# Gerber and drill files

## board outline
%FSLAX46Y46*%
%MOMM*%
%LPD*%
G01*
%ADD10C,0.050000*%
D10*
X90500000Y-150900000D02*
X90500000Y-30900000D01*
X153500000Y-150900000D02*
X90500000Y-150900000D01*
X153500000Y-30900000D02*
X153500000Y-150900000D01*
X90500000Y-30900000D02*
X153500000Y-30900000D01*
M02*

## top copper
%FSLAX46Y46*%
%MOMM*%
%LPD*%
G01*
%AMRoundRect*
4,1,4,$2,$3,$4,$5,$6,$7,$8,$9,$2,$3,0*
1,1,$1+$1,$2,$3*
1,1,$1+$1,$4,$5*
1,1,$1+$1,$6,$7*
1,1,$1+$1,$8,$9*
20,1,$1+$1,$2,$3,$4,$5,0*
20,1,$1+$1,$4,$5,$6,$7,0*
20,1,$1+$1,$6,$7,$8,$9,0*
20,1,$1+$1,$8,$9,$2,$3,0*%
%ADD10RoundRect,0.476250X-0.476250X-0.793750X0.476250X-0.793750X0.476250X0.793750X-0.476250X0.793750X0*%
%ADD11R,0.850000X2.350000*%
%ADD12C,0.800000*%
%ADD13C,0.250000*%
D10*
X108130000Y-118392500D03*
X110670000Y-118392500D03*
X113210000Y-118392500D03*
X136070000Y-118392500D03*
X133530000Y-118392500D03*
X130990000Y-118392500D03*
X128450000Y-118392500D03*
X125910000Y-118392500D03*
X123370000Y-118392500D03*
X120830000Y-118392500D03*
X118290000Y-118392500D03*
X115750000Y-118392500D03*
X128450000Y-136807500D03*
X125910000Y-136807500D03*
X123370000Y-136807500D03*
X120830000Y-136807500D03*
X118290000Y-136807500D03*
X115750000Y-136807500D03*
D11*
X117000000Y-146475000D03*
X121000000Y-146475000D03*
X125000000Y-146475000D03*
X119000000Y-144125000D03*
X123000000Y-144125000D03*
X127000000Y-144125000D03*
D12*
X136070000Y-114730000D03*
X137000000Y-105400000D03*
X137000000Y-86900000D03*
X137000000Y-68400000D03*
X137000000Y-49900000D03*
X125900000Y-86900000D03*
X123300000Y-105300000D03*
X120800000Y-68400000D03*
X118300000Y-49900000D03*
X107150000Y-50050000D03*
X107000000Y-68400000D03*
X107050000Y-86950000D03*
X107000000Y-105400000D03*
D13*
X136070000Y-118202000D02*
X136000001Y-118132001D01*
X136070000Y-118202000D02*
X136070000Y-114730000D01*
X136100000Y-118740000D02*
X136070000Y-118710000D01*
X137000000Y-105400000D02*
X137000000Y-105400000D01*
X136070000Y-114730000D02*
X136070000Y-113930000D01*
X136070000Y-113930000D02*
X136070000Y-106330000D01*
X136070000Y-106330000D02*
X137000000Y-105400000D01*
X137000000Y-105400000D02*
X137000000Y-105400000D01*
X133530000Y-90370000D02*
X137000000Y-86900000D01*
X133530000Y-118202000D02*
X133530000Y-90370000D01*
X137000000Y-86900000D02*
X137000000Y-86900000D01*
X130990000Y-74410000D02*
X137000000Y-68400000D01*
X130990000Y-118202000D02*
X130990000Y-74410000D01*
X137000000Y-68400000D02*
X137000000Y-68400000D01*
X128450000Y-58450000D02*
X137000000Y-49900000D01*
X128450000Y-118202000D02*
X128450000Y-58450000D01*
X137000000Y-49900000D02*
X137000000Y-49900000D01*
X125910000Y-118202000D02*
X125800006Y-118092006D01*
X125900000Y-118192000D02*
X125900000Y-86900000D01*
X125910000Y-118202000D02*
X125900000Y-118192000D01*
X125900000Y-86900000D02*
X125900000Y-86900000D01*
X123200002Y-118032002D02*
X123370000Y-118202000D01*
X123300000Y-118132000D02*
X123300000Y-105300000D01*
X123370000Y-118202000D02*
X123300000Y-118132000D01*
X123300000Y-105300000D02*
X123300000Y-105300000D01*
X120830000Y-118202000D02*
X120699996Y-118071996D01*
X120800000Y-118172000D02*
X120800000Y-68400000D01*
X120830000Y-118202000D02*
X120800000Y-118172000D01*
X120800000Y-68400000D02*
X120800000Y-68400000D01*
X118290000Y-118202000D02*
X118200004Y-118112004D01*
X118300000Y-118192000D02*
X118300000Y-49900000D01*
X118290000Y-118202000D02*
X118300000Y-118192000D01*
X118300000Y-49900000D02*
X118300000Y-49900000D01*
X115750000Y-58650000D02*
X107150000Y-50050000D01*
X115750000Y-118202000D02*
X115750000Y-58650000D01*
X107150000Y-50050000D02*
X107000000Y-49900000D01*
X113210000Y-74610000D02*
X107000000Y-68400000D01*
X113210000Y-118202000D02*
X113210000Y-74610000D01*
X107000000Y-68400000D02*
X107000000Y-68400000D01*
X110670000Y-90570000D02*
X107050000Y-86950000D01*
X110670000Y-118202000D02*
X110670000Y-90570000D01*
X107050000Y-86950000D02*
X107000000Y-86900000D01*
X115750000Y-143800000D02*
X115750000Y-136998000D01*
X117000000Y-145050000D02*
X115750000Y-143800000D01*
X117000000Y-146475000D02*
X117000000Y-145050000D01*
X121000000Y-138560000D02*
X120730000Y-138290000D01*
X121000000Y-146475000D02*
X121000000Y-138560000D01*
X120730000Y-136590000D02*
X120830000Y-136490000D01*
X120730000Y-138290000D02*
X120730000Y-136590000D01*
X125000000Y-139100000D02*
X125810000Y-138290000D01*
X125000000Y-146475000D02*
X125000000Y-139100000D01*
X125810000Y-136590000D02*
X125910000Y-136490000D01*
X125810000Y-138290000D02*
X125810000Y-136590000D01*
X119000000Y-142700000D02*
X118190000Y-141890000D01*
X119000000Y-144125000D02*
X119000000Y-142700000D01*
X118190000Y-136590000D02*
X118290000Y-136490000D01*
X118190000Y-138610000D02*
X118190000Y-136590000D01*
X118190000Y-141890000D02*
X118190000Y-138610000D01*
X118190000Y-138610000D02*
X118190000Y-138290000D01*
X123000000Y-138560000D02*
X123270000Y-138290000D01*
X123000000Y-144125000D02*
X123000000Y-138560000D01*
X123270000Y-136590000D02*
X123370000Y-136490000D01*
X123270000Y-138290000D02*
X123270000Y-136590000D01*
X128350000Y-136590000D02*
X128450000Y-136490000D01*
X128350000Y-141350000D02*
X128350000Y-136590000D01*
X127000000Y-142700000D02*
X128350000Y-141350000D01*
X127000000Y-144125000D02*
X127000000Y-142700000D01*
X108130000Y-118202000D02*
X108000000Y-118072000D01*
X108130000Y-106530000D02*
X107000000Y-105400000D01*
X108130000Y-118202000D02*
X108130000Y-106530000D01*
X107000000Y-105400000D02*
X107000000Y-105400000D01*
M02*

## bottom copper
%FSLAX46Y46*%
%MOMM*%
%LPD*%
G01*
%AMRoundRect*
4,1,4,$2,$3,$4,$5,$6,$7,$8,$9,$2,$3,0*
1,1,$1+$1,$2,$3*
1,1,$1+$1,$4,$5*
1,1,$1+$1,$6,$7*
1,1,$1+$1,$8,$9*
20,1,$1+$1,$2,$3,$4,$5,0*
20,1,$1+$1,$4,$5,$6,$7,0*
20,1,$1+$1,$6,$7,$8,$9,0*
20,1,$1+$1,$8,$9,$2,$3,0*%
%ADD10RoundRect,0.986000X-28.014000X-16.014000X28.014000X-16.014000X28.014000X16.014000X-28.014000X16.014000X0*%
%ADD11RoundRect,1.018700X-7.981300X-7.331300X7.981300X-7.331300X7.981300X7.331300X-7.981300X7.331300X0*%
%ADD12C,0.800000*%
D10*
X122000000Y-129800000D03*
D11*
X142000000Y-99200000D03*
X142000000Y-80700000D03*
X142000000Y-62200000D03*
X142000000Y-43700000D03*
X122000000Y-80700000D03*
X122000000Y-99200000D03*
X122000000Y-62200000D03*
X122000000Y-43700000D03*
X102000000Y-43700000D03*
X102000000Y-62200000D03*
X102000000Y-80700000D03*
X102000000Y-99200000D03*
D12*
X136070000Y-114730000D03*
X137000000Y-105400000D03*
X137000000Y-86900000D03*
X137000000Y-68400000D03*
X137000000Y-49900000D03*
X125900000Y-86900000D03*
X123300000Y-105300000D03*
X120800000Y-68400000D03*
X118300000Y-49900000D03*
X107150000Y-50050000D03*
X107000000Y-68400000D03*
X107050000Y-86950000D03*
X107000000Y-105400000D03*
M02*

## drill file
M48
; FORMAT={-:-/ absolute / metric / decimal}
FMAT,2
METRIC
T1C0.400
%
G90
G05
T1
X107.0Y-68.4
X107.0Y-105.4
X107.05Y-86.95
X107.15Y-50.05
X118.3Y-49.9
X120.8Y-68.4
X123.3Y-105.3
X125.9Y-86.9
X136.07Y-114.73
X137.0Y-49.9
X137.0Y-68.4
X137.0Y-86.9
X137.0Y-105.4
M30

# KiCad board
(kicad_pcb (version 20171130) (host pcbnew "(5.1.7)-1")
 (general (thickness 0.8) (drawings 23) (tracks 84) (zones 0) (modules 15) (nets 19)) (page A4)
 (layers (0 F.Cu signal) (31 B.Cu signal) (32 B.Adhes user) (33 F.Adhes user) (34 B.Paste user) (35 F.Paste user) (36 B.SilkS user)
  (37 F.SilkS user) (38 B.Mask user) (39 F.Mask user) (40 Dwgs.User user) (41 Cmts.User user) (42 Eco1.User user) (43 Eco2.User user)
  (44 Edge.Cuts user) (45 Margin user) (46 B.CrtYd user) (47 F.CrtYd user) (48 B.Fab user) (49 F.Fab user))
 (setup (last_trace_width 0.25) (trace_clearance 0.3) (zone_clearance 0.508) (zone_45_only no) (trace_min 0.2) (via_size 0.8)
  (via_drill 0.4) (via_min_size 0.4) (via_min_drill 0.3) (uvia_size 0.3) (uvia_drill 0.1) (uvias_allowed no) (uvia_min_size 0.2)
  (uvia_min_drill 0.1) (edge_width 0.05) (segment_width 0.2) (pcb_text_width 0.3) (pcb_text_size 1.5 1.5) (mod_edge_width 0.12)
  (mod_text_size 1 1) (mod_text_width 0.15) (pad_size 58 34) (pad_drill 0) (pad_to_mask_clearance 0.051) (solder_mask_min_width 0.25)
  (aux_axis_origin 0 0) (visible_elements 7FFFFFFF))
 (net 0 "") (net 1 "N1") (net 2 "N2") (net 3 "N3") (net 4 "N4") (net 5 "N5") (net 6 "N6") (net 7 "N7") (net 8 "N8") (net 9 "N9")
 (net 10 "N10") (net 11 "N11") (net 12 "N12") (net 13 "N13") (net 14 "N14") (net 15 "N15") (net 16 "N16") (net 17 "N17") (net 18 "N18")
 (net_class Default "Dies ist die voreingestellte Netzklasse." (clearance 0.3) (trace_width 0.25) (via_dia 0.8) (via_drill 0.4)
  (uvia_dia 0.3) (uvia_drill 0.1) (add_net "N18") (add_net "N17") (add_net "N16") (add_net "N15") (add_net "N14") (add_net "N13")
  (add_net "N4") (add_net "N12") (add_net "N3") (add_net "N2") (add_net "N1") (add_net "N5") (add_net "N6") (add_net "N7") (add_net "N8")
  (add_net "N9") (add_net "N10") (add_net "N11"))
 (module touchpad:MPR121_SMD (layer F.Cu) (at 122.1 127.6)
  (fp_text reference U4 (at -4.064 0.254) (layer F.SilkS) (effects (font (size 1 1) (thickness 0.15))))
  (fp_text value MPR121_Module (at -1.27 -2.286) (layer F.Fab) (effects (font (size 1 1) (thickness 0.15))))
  (pad 7 smd roundrect (at -13.97 -8.89) (size 1.905 2.54) (drill oval (offset 0 -0.3175)) (layers F.Cu F.Paste F.Mask)
   (roundrect_rratio 0.25) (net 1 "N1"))
  (pad 8 smd roundrect (at -11.43 -8.89) (size 1.905 2.54) (drill oval (offset 0 -0.3175)) (layers F.Cu F.Paste F.Mask)
   (roundrect_rratio 0.25) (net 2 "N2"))
  (pad 9 smd roundrect (at -8.89 -8.89) (size 1.905 2.54) (drill oval (offset 0 -0.3175)) (layers F.Cu F.Paste F.Mask)
   (roundrect_rratio 0.25) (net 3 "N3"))
  (pad 18 smd roundrect (at 13.97 -8.89) (size 1.905 2.54) (drill oval (offset 0 -0.3175)) (layers F.Cu F.Paste F.Mask)
   (roundrect_rratio 0.25) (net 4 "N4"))
  (pad 17 smd roundrect (at 11.43 -8.89) (size 1.905 2.54) (drill oval (offset 0 -0.3175)) (layers F.Cu F.Paste F.Mask)
   (roundrect_rratio 0.25) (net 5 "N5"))
  (pad 16 smd roundrect (at 8.89 -8.89) (size 1.905 2.54) (drill oval (offset 0 -0.3175)) (layers F.Cu F.Paste F.Mask)
   (roundrect_rratio 0.25) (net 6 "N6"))
  (pad 15 smd roundrect (at 6.35 -8.89) (size 1.905 2.54) (drill oval (offset 0 -0.3175)) (layers F.Cu F.Paste F.Mask)
   (roundrect_rratio 0.25) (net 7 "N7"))
  (pad 14 smd roundrect (at 3.81 -8.89) (size 1.905 2.54) (drill oval (offset 0 -0.3175)) (layers F.Cu F.Paste F.Mask)
   (roundrect_rratio 0.25) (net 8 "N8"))
  (pad 13 smd roundrect (at 1.27 -8.89) (size 1.905 2.54) (drill oval (offset 0 -0.3175)) (layers F.Cu F.Paste F.Mask)
   (roundrect_rratio 0.25) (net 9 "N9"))
  (pad 12 smd roundrect (at -1.27 -8.89) (size 1.905 2.54) (drill oval (offset 0 -0.3175)) (layers F.Cu F.Paste F.Mask)
   (roundrect_rratio 0.25) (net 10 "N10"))
  (pad 11 smd roundrect (at -3.81 -8.89) (size 1.905 2.54) (drill oval (offset 0 -0.3175)) (layers F.Cu F.Paste F.Mask)
   (roundrect_rratio 0.25) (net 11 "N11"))
  (pad 10 smd roundrect (at -6.35 -8.89) (size 1.905 2.54) (drill oval (offset 0 -0.3175)) (layers F.Cu F.Paste F.Mask)
   (roundrect_rratio 0.25) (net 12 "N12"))
  (pad 6 smd roundrect (at 6.35 8.89) (size 1.905 2.54) (drill oval (offset 0 0.3175)) (layers F.Cu F.Paste F.Mask) (roundrect_rratio 0.25)
   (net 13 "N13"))
  (pad 5 smd roundrect (at 3.81 8.89) (size 1.905 2.54) (drill oval (offset 0 0.3175)) (layers F.Cu F.Paste F.Mask) (roundrect_rratio 0.25)
   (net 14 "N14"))
  (pad 4 smd roundrect (at 1.27 8.89) (size 1.905 2.54) (drill oval (offset 0 0.3175)) (layers F.Cu F.Paste F.Mask) (roundrect_rratio 0.25)
   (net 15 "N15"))
  (pad 3 smd roundrect (at -1.27 8.89) (size 1.905 2.54) (drill oval (offset 0 0.3175)) (layers F.Cu F.Paste F.Mask) (roundrect_rratio 0.25)
   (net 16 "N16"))
  (pad 2 smd roundrect (at -3.81 8.89) (size 1.905 2.54) (drill oval (offset 0 0.3175)) (layers F.Cu F.Paste F.Mask) (roundrect_rratio 0.25)
   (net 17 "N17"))
  (pad 1 smd roundrect (at -6.35 8.89) (size 1.905 2.54) (drill oval (offset 0 0.3175)) (layers F.Cu F.Paste F.Mask) (roundrect_rratio 0.25)
   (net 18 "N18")))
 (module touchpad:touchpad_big (layer F.Cu) (at 122 129.8)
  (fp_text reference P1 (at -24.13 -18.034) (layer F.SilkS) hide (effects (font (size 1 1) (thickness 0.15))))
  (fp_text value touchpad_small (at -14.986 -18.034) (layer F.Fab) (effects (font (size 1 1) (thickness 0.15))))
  (pad 1 smd roundrect (at 0 0) (size 58 34) (layers B.Cu) (roundrect_rratio 0.029) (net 4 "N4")))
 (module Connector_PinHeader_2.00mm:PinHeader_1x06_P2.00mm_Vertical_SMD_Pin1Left (layer F.Cu) (at 122 145.3 90)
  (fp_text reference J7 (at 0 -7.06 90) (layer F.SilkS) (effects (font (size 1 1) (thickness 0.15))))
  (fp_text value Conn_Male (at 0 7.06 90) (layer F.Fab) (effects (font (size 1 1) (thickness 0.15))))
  (pad 1 smd rect (at -1.175 -5 90) (size 2.35 0.85) (layers F.Cu F.Paste F.Mask) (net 18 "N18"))
  (pad 3 smd rect (at -1.175 -1 90) (size 2.35 0.85) (layers F.Cu F.Paste F.Mask) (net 16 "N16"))
  (pad 5 smd rect (at -1.175 3 90) (size 2.35 0.85) (layers F.Cu F.Paste F.Mask) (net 14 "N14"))
  (pad 2 smd rect (at 1.175 -3 90) (size 2.35 0.85) (layers F.Cu F.Paste F.Mask) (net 17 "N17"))
  (pad 4 smd rect (at 1.175 1 90) (size 2.35 0.85) (layers F.Cu F.Paste F.Mask) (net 15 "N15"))
  (pad 6 smd rect (at 1.175 5 90) (size 2.35 0.85) (layers F.Cu F.Paste F.Mask) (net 13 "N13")))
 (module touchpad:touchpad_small (layer F.Cu) (at 142 99.2)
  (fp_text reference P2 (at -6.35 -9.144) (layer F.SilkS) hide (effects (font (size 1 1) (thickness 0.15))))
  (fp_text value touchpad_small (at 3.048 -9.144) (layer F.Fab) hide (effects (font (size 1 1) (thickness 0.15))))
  (pad 1 smd roundrect (at 0 0) (size 18 16.7) (layers B.Cu) (roundrect_rratio 0.061) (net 4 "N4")))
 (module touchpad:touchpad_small (layer F.Cu) (at 142 80.7)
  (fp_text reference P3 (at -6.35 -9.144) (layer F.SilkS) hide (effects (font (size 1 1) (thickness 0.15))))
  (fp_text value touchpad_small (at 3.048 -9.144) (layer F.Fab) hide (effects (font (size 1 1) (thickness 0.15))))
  (pad 1 smd roundrect (at 0 0) (size 18 16.7) (layers B.Cu) (roundrect_rratio 0.061) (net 5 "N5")))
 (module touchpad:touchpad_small (layer F.Cu) (at 142 62.2)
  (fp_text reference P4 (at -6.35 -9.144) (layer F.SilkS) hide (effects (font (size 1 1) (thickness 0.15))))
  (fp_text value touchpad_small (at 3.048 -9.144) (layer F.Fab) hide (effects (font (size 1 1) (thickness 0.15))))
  (pad 1 smd roundrect (at 0 0) (size 18 16.7) (layers B.Cu) (roundrect_rratio 0.061) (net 6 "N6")))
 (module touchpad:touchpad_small (layer F.Cu) (at 142 43.7)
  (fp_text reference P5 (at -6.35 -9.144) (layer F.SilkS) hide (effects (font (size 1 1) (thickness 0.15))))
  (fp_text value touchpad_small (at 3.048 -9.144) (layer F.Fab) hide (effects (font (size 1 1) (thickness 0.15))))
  (pad 1 smd roundrect (at 0 0) (size 18 16.7) (layers B.Cu) (roundrect_rratio 0.061) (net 7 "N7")))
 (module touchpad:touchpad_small (layer F.Cu) (at 122 80.7)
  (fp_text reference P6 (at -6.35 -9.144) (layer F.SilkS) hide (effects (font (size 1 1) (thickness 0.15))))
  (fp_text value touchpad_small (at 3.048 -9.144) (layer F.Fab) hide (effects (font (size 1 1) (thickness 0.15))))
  (pad 1 smd roundrect (at 0 0) (size 18 16.7) (layers B.Cu) (roundrect_rratio 0.061) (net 8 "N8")))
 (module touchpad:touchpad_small (layer F.Cu) (at 122 99.2)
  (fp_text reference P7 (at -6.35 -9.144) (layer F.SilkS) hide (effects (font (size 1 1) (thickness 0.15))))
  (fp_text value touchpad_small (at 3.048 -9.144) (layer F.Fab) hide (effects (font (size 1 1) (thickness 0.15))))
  (pad 1 smd roundrect (at 0 0) (size 18 16.7) (layers B.Cu) (roundrect_rratio 0.061) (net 9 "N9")))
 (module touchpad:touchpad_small (layer F.Cu) (at 122 62.2)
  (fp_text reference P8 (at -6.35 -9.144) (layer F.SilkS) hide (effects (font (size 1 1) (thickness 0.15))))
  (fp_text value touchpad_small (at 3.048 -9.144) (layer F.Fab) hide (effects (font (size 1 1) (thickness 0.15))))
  (pad 1 smd roundrect (at 0 0) (size 18 16.7) (layers B.Cu) (roundrect_rratio 0.061) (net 10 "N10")))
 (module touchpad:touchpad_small (layer F.Cu) (at 122 43.7)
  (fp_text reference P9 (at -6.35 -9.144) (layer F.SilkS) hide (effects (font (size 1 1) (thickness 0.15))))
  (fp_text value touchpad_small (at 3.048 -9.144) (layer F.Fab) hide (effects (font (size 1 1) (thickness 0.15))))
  (pad 1 smd roundrect (at 0 0) (size 18 16.7) (layers B.Cu) (roundrect_rratio 0.061) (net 11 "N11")))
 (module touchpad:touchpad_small (layer F.Cu) (at 102 43.7)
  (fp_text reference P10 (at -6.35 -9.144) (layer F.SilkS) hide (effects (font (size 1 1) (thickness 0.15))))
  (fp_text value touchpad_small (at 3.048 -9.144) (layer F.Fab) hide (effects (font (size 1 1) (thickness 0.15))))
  (pad 1 smd roundrect (at 0 0) (size 18 16.7) (layers B.Cu) (roundrect_rratio 0.061) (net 12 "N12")))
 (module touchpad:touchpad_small (layer F.Cu) (at 102 62.2)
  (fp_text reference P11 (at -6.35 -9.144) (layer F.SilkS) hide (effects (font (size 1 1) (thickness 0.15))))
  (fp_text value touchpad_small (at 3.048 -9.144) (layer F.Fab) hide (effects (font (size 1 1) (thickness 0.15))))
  (pad 1 smd roundrect (at 0 0) (size 18 16.7) (layers B.Cu) (roundrect_rratio 0.061) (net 3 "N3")))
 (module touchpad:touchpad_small (layer F.Cu) (at 102 80.7)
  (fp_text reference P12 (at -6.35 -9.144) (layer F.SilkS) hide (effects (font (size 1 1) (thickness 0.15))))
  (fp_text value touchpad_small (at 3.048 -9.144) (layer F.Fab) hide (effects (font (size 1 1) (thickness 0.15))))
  (pad 1 smd roundrect (at 0 0) (size 18 16.7) (layers B.Cu) (roundrect_rratio 0.061) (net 2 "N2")))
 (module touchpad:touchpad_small (layer F.Cu) (at 102 99.2)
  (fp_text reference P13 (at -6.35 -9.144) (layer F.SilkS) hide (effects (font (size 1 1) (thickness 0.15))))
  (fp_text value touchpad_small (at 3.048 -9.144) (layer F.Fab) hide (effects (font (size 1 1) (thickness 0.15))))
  (pad 1 smd roundrect (at 0 0) (size 18 16.7) (layers B.Cu) (roundrect_rratio 0.061) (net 1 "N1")))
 (gr_line (start 90.5 150.9) (end 90.5 30.9) (layer Edge.Cuts) (width 0.05))
 (gr_line (start 153.5 150.9) (end 90.5 150.9) (layer Edge.Cuts) (width 0.05))
 (gr_line (start 153.5 30.9) (end 153.5 150.9) (layer Edge.Cuts) (width 0.05))
 (gr_line (start 90.5 30.9) (end 153.5 30.9) (layer Edge.Cuts) (width 0.05))
 (segment (start 136.07 118.202) (end 136.000001 118.132001) (width 0.25) (layer F.Cu) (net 4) (status 30))
 (segment (start 136.07 118.202) (end 136.07 114.73) (width 0.25) (layer F.Cu) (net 4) (status 10))
 (segment (start 136.1 118.74) (end 136.07 118.71) (width 0.25) (layer F.Cu) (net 4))
 (segment (start 137 105.4) (end 137 105.4) (width 0.25) (layer F.Cu) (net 4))
 (via (at 136.07 114.73) (size 0.8) (drill 0.4) (layers F.Cu B.Cu) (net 4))
 (segment (start 136.07 114.73) (end 136.07 113.93) (width 0.25) (layer F.Cu) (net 4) (status 10))
 (segment (start 136.07 113.93) (end 136.07 106.33) (width 0.25) (layer F.Cu) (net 4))
 (segment (start 136.07 106.33) (end 137 105.4) (width 0.25) (layer F.Cu) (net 4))
 (segment (start 137 105.4) (end 137 105.4) (width 0.25) (layer F.Cu) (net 4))
 (via (at 137 105.4) (size 0.8) (drill 0.4) (layers F.Cu B.Cu) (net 4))
 (segment (start 133.53 90.37) (end 137 86.9) (width 0.25) (layer F.Cu) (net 5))
 (segment (start 133.53 118.202) (end 133.53 90.37) (width 0.25) (layer F.Cu) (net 5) (status 10))
 (segment (start 137 86.9) (end 137 86.9) (width 0.25) (layer F.Cu) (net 5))
 (via (at 137 86.9) (size 0.8) (drill 0.4) (layers F.Cu B.Cu) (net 5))
 (segment (start 130.99 74.41) (end 137 68.4) (width 0.25) (layer F.Cu) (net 6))
 (segment (start 130.99 118.202) (end 130.99 74.41) (width 0.25) (layer F.Cu) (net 6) (status 10))
 (segment (start 137 68.4) (end 137 68.4) (width 0.25) (layer F.Cu) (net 6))
 (via (at 137 68.4) (size 0.8) (drill 0.4) (layers F.Cu B.Cu) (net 6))
 (segment (start 128.45 58.45) (end 137 49.9) (width 0.25) (layer F.Cu) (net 7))
 (segment (start 128.45 118.202) (end 128.45 58.45) (width 0.25) (layer F.Cu) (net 7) (status 10))
 (segment (start 137 49.9) (end 137 49.9) (width 0.25) (layer F.Cu) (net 7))
 (via (at 137 49.9) (size 0.8) (drill 0.4) (layers F.Cu B.Cu) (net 7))
 (segment (start 125.91 118.202) (end 125.800006 118.092006) (width 0.25) (layer F.Cu) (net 8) (status 30))
 (segment (start 125.9 118.192) (end 125.9 86.9) (width 0.25) (layer F.Cu) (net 8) (status 10))
 (segment (start 125.91 118.202) (end 125.9 118.192) (width 0.25) (layer F.Cu) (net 8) (status 30))
 (segment (start 125.9 86.9) (end 125.9 86.9) (width 0.25) (layer F.Cu) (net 8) (status 10))
 (via (at 125.9 86.9) (size 0.8) (drill 0.4) (layers F.Cu B.Cu) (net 8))
 (segment (start 123.200002 118.032002) (end 123.37 118.202) (width 0.25) (layer F.Cu) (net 9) (status 30))
 (segment (start 123.3 118.132) (end 123.3 105.3) (width 0.25) (layer F.Cu) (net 9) (status 10))
 (segment (start 123.37 118.202) (end 123.3 118.132) (width 0.25) (layer F.Cu) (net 9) (status 30))
 (segment (start 123.3 105.3) (end 123.3 105.3) (width 0.25) (layer F.Cu) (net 9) (status 10))
 (via (at 123.3 105.3) (size 0.8) (drill 0.4) (layers F.Cu B.Cu) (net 9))
 (segment (start 120.83 118.202) (end 120.699996 118.071996) (width 0.25) (layer F.Cu) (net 10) (status 30))
 (segment (start 120.8 118.172) (end 120.8 68.4) (width 0.25) (layer F.Cu) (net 10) (status 10))
 (segment (start 120.83 118.202) (end 120.8 118.172) (width 0.25) (layer F.Cu) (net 10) (status 30))
 (segment (start 120.8 68.4) (end 120.8 68.4) (width 0.25) (layer F.Cu) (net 10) (status 10))
 (via (at 120.8 68.4) (size 0.8) (drill 0.4) (layers F.Cu B.Cu) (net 10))
 (segment (start 118.29 118.202) (end 118.200004 118.112004) (width 0.25) (layer F.Cu) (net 11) (status 30))
 (segment (start 118.3 118.192) (end 118.3 49.9) (width 0.25) (layer F.Cu) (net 11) (status 10))
 (segment (start 118.29 118.202) (end 118.3 118.192) (width 0.25) (layer F.Cu) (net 11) (status 30))
 (segment (start 118.3 49.9) (end 118.3 49.9) (width 0.25) (layer F.Cu) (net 11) (status 10))
 (via (at 118.3 49.9) (size 0.8) (drill 0.4) (layers F.Cu B.Cu) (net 11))
 (segment (start 115.75 58.65) (end 107.15 50.05) (width 0.25) (layer F.Cu) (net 12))
 (segment (start 115.75 118.202) (end 115.75 58.65) (width 0.25) (layer F.Cu) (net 12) (status 10))
 (segment (start 107.15 50.05) (end 107 49.9) (width 0.25) (layer F.Cu) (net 12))
 (via (at 107.15 50.05) (size 0.8) (drill 0.4) (layers F.Cu B.Cu) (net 12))
 (segment (start 113.21 74.61) (end 107 68.4) (width 0.25) (layer F.Cu) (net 3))
 (segment (start 113.21 118.202) (end 113.21 74.61) (width 0.25) (layer F.Cu) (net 3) (status 10))
 (segment (start 107 68.4) (end 107 68.4) (width 0.25) (layer F.Cu) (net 3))
 (via (at 107 68.4) (size 0.8) (drill 0.4) (layers F.Cu B.Cu) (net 3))
 (segment (start 110.67 90.57) (end 107.05 86.95) (width 0.25) (layer F.Cu) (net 2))
 (segment (start 110.67 118.202) (end 110.67 90.57) (width 0.25) (layer F.Cu) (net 2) (status 10))
 (segment (start 107.05 86.95) (end 107 86.9) (width 0.25) (layer F.Cu) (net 2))
 (via (at 107.05 86.95) (size 0.8) (drill 0.4) (layers F.Cu B.Cu) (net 2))
 (segment (start 115.75 143.8) (end 115.75 136.998) (width 0.25) (layer F.Cu) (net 18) (status 20))
 (segment (start 117 145.05) (end 115.75 143.8) (width 0.25) (layer F.Cu) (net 18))
 (segment (start 117 146.475) (end 117 145.05) (width 0.25) (layer F.Cu) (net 18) (status 10))
 (segment (start 121 138.56) (end 120.73 138.29) (width 0.25) (layer F.Cu) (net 16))
 (segment (start 121 146.475) (end 121 138.56) (width 0.25) (layer F.Cu) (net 16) (status 10))
 (segment (start 120.73 136.59) (end 120.83 136.49) (width 0.25) (layer F.Cu) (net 16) (status 30))
 (segment (start 120.73 138.29) (end 120.73 136.59) (width 0.25) (layer F.Cu) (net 16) (status 20))
 (segment (start 125 139.1) (end 125.81 138.29) (width 0.25) (layer F.Cu) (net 14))
 (segment (start 125 146.475) (end 125 139.1) (width 0.25) (layer F.Cu) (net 14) (status 10))
 (segment (start 125.81 136.59) (end 125.91 136.49) (width 0.25) (layer F.Cu) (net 14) (status 30))
 (segment (start 125.81 138.29) (end 125.81 136.59) (width 0.25) (layer F.Cu) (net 14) (status 20))
 (segment (start 119 142.7) (end 118.19 141.89) (width 0.25) (layer F.Cu) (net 17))
 (segment (start 119 144.125) (end 119 142.7) (width 0.25) (layer F.Cu) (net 17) (status 10))
 (segment (start 118.19 136.59) (end 118.29 136.49) (width 0.25) (layer F.Cu) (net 17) (status 30))
 (segment (start 118.19 138.61) (end 118.19 136.59) (width 0.25) (layer F.Cu) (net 17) (status 20))
 (segment (start 118.19 141.89) (end 118.19 138.61) (width 0.25) (layer F.Cu) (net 17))
 (segment (start 118.19 138.61) (end 118.19 138.29) (width 0.25) (layer F.Cu) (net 17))
 (segment (start 123 138.56) (end 123.27 138.29) (width 0.25) (layer F.Cu) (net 15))
 (segment (start 123 144.125) (end 123 138.56) (width 0.25) (layer F.Cu) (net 15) (status 10))
 (segment (start 123.27 136.59) (end 123.37 136.49) (width 0.25) (layer F.Cu) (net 15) (status 30))
 (segment (start 123.27 138.29) (end 123.27 136.59) (width 0.25) (layer F.Cu) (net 15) (status 20))
 (segment (start 128.35 136.59) (end 128.45 136.49) (width 0.25) (layer F.Cu) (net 13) (status 30))
 (segment (start 128.35 141.35) (end 128.35 136.59) (width 0.25) (layer F.Cu) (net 13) (status 20))
 (segment (start 127 142.7) (end 128.35 141.35) (width 0.25) (layer F.Cu) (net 13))
 (segment (start 127 144.125) (end 127 142.7) (width 0.25) (layer F.Cu) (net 13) (status 10))
 (segment (start 108.13 118.202) (end 108 118.072) (width 0.25) (layer F.Cu) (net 1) (status 30))
 (segment (start 108.13 106.53) (end 107 105.4) (width 0.25) (layer F.Cu) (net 1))
 (segment (start 108.13 118.202) (end 108.13 106.53) (width 0.25) (layer F.Cu) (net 1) (status 10))
 (segment (start 107 105.4) (end 107 105.4) (width 0.25) (layer F.Cu) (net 1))
 (via (at 107 105.4) (size 0.8) (drill 0.4) (layers F.Cu B.Cu) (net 1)))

